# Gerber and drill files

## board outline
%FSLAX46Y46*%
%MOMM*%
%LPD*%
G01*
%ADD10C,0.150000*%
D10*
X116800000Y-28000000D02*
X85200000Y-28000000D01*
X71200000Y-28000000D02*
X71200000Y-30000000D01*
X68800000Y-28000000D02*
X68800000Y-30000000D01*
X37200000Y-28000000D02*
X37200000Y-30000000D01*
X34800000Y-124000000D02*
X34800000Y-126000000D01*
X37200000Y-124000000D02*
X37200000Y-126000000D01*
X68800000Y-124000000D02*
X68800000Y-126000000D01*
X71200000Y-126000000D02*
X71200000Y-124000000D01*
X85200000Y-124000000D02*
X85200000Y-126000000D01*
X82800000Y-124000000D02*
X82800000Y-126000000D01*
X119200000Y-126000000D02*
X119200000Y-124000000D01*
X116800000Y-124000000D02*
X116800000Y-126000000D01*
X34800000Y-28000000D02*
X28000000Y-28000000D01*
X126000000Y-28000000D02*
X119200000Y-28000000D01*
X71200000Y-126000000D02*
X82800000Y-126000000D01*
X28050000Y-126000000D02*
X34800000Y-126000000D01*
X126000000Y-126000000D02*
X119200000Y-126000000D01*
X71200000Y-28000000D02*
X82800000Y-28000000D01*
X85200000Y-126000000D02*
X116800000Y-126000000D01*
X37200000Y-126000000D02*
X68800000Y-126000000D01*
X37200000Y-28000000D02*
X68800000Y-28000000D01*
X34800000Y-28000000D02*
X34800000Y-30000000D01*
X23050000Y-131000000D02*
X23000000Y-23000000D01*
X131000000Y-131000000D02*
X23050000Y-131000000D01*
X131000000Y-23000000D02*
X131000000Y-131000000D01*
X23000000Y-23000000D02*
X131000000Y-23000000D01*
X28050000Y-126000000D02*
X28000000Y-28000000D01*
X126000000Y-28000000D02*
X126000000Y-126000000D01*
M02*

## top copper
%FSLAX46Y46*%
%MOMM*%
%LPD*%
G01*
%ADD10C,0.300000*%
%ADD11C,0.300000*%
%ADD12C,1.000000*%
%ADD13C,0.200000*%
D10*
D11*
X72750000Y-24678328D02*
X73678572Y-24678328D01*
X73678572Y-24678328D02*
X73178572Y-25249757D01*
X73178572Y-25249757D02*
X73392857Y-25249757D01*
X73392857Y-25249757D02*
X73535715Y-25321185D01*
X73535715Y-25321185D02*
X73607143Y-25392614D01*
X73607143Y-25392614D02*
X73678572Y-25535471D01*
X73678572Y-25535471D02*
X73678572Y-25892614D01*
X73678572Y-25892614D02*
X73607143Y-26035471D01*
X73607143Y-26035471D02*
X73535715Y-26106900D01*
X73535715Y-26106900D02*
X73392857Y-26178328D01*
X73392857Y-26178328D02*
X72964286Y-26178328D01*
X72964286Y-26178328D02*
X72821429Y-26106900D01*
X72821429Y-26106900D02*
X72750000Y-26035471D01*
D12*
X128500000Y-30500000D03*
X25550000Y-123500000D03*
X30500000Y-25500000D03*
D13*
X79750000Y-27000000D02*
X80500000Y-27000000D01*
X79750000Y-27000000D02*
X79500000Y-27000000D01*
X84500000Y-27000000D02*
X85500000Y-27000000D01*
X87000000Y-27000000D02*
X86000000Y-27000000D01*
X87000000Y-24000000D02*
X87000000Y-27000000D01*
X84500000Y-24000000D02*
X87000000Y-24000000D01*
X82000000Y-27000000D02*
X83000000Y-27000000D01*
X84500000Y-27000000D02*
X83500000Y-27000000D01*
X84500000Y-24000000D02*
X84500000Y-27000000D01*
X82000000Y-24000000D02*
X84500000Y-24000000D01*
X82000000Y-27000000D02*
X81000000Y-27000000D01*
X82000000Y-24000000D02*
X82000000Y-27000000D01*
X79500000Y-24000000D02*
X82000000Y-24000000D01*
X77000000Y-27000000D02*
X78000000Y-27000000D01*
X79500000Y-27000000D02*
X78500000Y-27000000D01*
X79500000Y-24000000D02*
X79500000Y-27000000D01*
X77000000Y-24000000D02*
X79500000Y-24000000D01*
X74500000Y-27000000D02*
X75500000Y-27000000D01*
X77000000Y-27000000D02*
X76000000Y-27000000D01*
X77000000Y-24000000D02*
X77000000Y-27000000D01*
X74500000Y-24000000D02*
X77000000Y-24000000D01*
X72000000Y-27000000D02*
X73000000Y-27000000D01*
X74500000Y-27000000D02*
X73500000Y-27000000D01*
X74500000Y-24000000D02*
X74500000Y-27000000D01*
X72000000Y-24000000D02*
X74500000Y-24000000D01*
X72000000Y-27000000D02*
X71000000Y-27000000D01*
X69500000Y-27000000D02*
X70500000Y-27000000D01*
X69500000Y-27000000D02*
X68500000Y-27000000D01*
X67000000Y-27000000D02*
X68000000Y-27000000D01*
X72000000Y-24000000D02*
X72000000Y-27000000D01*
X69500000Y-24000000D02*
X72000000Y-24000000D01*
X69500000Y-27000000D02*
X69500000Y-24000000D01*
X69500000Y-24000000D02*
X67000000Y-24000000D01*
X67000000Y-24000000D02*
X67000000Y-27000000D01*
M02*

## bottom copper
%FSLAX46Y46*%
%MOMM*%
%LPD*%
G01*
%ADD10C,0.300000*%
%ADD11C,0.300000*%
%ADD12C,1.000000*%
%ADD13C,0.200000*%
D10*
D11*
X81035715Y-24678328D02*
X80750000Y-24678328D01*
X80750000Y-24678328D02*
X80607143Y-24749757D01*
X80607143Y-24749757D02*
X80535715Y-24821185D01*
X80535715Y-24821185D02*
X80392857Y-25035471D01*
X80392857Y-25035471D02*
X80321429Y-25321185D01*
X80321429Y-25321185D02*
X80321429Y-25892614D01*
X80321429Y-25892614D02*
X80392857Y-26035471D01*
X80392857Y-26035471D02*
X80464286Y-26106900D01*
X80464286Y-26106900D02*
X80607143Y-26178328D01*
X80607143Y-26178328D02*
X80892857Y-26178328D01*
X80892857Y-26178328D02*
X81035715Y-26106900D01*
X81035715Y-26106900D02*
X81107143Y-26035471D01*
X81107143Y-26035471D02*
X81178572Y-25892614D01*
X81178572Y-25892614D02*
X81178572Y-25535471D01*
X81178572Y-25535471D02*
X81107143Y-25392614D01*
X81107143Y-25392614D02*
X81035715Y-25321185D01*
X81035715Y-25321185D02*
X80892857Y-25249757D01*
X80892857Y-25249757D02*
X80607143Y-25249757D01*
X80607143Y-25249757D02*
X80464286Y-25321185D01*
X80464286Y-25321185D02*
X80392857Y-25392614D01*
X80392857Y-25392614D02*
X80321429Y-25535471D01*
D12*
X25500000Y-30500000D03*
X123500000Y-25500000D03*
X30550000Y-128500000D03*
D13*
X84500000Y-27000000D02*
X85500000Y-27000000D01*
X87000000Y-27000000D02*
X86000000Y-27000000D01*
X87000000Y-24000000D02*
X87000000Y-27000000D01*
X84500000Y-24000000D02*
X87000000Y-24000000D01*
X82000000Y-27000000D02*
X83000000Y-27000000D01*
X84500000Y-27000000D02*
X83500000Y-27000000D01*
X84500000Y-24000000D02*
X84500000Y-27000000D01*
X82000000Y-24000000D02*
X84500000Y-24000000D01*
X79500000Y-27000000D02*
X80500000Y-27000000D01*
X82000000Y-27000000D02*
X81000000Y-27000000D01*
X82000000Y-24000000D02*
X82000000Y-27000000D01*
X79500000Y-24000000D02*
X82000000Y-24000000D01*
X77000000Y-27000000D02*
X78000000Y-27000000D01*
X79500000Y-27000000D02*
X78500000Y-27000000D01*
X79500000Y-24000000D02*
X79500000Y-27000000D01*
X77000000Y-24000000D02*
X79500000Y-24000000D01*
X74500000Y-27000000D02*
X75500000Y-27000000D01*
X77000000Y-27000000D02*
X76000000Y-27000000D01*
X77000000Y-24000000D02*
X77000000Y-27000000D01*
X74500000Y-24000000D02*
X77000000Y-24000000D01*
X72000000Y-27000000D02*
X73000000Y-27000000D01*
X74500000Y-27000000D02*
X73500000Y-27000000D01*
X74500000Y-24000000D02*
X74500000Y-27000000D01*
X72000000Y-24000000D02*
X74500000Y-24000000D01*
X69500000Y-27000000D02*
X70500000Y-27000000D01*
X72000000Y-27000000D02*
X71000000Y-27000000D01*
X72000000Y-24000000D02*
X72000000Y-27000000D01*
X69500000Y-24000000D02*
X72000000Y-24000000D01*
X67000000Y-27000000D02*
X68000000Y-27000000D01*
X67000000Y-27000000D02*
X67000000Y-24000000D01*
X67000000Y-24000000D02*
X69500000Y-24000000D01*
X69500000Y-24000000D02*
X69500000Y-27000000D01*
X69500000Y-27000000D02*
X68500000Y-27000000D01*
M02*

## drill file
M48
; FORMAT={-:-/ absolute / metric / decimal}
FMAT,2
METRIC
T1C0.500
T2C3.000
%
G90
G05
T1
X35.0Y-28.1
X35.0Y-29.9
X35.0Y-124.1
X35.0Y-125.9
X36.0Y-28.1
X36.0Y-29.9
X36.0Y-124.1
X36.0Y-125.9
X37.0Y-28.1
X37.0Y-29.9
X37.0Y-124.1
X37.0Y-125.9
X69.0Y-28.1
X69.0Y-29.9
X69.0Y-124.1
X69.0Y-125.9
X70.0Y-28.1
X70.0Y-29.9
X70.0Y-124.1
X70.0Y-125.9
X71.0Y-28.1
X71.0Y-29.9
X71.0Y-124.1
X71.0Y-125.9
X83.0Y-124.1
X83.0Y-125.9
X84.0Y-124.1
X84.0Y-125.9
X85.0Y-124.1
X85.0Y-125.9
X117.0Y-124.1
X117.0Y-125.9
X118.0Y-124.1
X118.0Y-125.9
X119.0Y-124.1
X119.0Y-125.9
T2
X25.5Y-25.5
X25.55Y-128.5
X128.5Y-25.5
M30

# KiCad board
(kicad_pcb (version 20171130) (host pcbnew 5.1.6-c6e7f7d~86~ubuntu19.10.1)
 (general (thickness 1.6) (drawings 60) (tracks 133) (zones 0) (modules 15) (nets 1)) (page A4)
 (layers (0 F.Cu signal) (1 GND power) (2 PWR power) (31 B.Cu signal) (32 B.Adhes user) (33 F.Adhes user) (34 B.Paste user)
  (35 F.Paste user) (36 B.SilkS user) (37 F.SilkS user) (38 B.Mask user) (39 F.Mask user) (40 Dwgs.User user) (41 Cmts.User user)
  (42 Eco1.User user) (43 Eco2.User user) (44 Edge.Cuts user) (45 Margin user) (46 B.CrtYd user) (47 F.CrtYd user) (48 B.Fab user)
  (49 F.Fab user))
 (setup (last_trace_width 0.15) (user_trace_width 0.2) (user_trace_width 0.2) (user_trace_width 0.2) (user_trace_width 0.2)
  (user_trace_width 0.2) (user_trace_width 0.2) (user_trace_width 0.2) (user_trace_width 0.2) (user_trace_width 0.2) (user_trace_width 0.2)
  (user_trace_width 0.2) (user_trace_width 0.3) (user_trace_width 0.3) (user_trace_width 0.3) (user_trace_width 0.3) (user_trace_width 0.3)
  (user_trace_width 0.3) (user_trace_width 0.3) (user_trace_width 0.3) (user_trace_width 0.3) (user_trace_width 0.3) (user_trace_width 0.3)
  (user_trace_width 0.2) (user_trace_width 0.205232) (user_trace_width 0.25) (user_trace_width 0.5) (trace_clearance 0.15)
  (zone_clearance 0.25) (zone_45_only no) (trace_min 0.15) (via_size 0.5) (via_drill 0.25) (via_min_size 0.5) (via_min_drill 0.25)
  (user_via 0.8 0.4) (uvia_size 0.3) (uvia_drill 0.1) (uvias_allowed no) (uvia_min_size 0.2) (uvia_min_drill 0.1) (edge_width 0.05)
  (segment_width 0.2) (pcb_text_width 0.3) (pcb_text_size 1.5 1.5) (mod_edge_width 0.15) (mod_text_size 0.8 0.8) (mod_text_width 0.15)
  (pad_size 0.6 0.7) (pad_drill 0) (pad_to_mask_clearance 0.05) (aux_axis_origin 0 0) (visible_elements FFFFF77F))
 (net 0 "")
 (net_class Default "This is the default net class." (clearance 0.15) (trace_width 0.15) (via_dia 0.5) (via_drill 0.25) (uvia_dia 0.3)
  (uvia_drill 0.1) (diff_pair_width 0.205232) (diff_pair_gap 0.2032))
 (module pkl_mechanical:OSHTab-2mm (layer F.Cu) (at 36 125)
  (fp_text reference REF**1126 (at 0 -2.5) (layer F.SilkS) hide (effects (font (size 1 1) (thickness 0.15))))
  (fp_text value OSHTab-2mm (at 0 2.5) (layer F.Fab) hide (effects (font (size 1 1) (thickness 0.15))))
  (pad "" np_thru_hole circle (at 1 0.9) (size 0.5 0.5) (drill 0.5) (layers *.Cu))
  (pad "" np_thru_hole circle (at 0 0.9) (size 0.5 0.5) (drill 0.5) (layers *.Cu))
  (pad "" np_thru_hole circle (at -1 0.9) (size 0.5 0.5) (drill 0.5) (layers *.Cu))
  (pad "" np_thru_hole circle (at 1 -0.9) (size 0.5 0.5) (drill 0.5) (layers *.Cu))
  (pad "" np_thru_hole circle (at -1 -0.9) (size 0.5 0.5) (drill 0.5) (layers *.Cu))
  (pad "" np_thru_hole circle (at 0 -0.9) (size 0.5 0.5) (drill 0.5) (layers *.Cu)))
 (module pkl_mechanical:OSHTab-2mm (layer F.Cu) (at 70 125)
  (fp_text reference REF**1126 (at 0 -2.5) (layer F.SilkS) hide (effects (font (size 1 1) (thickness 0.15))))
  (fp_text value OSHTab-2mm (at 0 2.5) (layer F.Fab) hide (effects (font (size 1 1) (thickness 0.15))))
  (pad "" np_thru_hole circle (at 1 0.9) (size 0.5 0.5) (drill 0.5) (layers *.Cu))
  (pad "" np_thru_hole circle (at 0 0.9) (size 0.5 0.5) (drill 0.5) (layers *.Cu))
  (pad "" np_thru_hole circle (at -1 0.9) (size 0.5 0.5) (drill 0.5) (layers *.Cu))
  (pad "" np_thru_hole circle (at 1 -0.9) (size 0.5 0.5) (drill 0.5) (layers *.Cu))
  (pad "" np_thru_hole circle (at -1 -0.9) (size 0.5 0.5) (drill 0.5) (layers *.Cu))
  (pad "" np_thru_hole circle (at 0 -0.9) (size 0.5 0.5) (drill 0.5) (layers *.Cu)))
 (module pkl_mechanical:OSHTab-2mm (layer F.Cu) (at 84 125)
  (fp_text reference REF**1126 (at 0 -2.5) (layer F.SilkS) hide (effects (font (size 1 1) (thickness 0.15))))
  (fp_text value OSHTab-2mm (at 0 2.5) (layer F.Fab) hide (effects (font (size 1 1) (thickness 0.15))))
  (pad "" np_thru_hole circle (at 1 0.9) (size 0.5 0.5) (drill 0.5) (layers *.Cu))
  (pad "" np_thru_hole circle (at 0 0.9) (size 0.5 0.5) (drill 0.5) (layers *.Cu))
  (pad "" np_thru_hole circle (at -1 0.9) (size 0.5 0.5) (drill 0.5) (layers *.Cu))
  (pad "" np_thru_hole circle (at 1 -0.9) (size 0.5 0.5) (drill 0.5) (layers *.Cu))
  (pad "" np_thru_hole circle (at -1 -0.9) (size 0.5 0.5) (drill 0.5) (layers *.Cu))
  (pad "" np_thru_hole circle (at 0 -0.9) (size 0.5 0.5) (drill 0.5) (layers *.Cu)))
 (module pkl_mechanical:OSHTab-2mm (layer F.Cu) (at 118 125)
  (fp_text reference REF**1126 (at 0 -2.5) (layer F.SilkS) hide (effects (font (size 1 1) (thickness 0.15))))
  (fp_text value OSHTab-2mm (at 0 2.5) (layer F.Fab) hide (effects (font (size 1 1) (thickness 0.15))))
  (pad "" np_thru_hole circle (at 1 0.9) (size 0.5 0.5) (drill 0.5) (layers *.Cu))
  (pad "" np_thru_hole circle (at 0 0.9) (size 0.5 0.5) (drill 0.5) (layers *.Cu))
  (pad "" np_thru_hole circle (at -1 0.9) (size 0.5 0.5) (drill 0.5) (layers *.Cu))
  (pad "" np_thru_hole circle (at 1 -0.9) (size 0.5 0.5) (drill 0.5) (layers *.Cu))
  (pad "" np_thru_hole circle (at -1 -0.9) (size 0.5 0.5) (drill 0.5) (layers *.Cu))
  (pad "" np_thru_hole circle (at 0 -0.9) (size 0.5 0.5) (drill 0.5) (layers *.Cu)))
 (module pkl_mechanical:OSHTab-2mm (layer F.Cu) (at 70 29)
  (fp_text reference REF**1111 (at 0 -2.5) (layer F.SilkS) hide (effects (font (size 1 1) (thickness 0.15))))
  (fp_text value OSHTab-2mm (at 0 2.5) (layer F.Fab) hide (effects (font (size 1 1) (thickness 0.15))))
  (pad "" np_thru_hole circle (at 1 0.9) (size 0.5 0.5) (drill 0.5) (layers *.Cu))
  (pad "" np_thru_hole circle (at 0 0.9) (size 0.5 0.5) (drill 0.5) (layers *.Cu))
  (pad "" np_thru_hole circle (at -1 0.9) (size 0.5 0.5) (drill 0.5) (layers *.Cu))
  (pad "" np_thru_hole circle (at 1 -0.9) (size 0.5 0.5) (drill 0.5) (layers *.Cu))
  (pad "" np_thru_hole circle (at -1 -0.9) (size 0.5 0.5) (drill 0.5) (layers *.Cu))
  (pad "" np_thru_hole circle (at 0 -0.9) (size 0.5 0.5) (drill 0.5) (layers *.Cu)))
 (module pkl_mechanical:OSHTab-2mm (layer F.Cu) (at 36 29)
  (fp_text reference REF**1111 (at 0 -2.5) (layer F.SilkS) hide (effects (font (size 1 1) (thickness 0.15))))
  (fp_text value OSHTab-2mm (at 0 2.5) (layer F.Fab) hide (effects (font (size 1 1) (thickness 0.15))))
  (pad "" np_thru_hole circle (at 1 0.9) (size 0.5 0.5) (drill 0.5) (layers *.Cu))
  (pad "" np_thru_hole circle (at 0 0.9) (size 0.5 0.5) (drill 0.5) (layers *.Cu))
  (pad "" np_thru_hole circle (at -1 0.9) (size 0.5 0.5) (drill 0.5) (layers *.Cu))
  (pad "" np_thru_hole circle (at 1 -0.9) (size 0.5 0.5) (drill 0.5) (layers *.Cu))
  (pad "" np_thru_hole circle (at -1 -0.9) (size 0.5 0.5) (drill 0.5) (layers *.Cu))
  (pad "" np_thru_hole circle (at 0 -0.9) (size 0.5 0.5) (drill 0.5) (layers *.Cu)))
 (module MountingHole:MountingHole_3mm (layer F.Cu) (at 25.5 25.5)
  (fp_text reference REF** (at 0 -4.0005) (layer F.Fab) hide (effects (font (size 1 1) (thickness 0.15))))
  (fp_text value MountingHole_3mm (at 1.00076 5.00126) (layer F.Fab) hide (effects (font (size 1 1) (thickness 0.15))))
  (pad 1 np_thru_hole circle (at 0 0) (size 3 3) (drill 3) (layers *.Cu *.Mask)))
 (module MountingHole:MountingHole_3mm (layer F.Cu) (at 25.55 128.5)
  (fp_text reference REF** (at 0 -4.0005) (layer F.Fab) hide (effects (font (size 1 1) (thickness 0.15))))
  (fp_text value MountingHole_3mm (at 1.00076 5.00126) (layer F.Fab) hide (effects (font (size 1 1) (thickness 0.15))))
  (pad 1 np_thru_hole circle (at 0 0) (size 3 3) (drill 3) (layers *.Cu *.Mask)))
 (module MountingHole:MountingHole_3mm (layer F.Cu) (at 128.5 25.5)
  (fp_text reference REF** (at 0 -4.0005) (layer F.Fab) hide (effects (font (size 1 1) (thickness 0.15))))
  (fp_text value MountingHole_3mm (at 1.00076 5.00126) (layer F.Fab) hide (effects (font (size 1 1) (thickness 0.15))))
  (pad 1 np_thru_hole circle (at 0 0) (size 3 3) (drill 3) (layers *.Cu *.Mask)))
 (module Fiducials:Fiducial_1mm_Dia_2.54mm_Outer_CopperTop (layer B.Cu) (at 25.5 30.5)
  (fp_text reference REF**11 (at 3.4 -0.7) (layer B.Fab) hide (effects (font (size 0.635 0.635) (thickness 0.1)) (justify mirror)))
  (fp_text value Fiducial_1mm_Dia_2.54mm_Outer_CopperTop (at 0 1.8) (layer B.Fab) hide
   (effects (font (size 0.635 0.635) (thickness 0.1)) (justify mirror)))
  (pad ~ smd circle (at 0 0) (size 1 1) (layers B.Cu B.Mask) (solder_mask_margin 0.77) (clearance 0.77)))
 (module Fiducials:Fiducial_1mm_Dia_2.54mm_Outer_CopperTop (layer B.Cu) (at 123.5 25.5)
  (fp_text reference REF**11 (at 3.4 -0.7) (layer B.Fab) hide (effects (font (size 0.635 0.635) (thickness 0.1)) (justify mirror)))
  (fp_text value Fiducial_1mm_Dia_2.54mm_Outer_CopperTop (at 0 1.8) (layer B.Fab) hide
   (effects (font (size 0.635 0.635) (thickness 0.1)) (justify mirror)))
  (pad ~ smd circle (at 0 0) (size 1 1) (layers B.Cu B.Mask) (solder_mask_margin 0.77) (clearance 0.77)))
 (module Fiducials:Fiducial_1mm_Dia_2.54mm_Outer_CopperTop (layer B.Cu) (at 30.55 128.5)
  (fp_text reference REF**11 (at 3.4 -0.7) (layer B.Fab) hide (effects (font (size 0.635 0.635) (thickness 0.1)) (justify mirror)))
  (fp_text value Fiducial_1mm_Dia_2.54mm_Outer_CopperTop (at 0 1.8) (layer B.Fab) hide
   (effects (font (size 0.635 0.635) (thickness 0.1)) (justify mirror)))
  (pad ~ smd circle (at 0 0) (size 1 1) (layers B.Cu B.Mask) (solder_mask_margin 0.77) (clearance 0.77)))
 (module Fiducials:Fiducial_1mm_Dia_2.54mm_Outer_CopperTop (layer F.Cu) (at 128.5 30.5)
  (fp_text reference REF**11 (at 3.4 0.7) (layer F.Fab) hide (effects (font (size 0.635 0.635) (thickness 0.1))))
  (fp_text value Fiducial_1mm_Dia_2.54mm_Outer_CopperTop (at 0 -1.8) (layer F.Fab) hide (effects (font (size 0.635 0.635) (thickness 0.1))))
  (pad ~ smd circle (at 0 0) (size 1 1) (layers F.Cu F.Mask) (solder_mask_margin 0.77) (clearance 0.77)))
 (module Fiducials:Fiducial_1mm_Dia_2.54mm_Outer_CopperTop (layer F.Cu) (at 25.55 123.5)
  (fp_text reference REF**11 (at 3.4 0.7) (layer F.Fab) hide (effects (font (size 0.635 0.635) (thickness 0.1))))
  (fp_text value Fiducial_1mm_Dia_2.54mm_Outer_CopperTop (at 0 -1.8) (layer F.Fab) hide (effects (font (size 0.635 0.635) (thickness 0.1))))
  (pad ~ smd circle (at 0 0) (size 1 1) (layers F.Cu F.Mask) (solder_mask_margin 0.77) (clearance 0.77)))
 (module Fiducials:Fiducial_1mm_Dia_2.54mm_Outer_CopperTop (layer F.Cu) (at 30.5 25.5)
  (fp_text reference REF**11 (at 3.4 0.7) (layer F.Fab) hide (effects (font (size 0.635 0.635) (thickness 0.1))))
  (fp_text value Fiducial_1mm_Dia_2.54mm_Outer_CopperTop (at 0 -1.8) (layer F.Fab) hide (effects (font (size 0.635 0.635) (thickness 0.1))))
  (pad ~ smd circle (at 0 0) (size 1 1) (layers F.Cu F.Mask) (solder_mask_margin 0.77) (clearance 0.77)))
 (gr_line (start 116.8 28) (end 85.2 28) (layer Edge.Cuts) (width 0.15))
 (gr_line (start 71.2 28) (end 71.2 30) (layer Edge.Cuts) (width 0.15))
 (gr_line (start 68.8 28) (end 68.8 30) (layer Edge.Cuts) (width 0.15))
 (gr_line (start 37.2 28) (end 37.2 30) (layer Edge.Cuts) (width 0.15))
 (gr_line (start 34.8 124) (end 34.8 126) (layer Edge.Cuts) (width 0.15))
 (gr_line (start 37.2 124) (end 37.2 126) (layer Edge.Cuts) (width 0.15))
 (gr_line (start 68.8 124) (end 68.8 126) (layer Edge.Cuts) (width 0.15))
 (gr_line (start 71.2 126) (end 71.2 124) (layer Edge.Cuts) (width 0.15))
 (gr_line (start 85.2 124) (end 85.2 126) (layer Edge.Cuts) (width 0.15))
 (gr_line (start 82.8 124) (end 82.8 126) (layer Edge.Cuts) (width 0.15))
 (gr_line (start 119.2 126) (end 119.2 124) (layer Edge.Cuts) (width 0.15))
 (gr_line (start 116.8 124) (end 116.8 126) (layer Edge.Cuts) (width 0.15))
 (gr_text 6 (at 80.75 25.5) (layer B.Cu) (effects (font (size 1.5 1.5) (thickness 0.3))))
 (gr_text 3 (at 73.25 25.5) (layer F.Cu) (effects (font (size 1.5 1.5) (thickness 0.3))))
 (gr_line (start 34.8 28) (end 28 28) (layer Edge.Cuts) (width 0.15))
 (gr_line (start 126 28) (end 119.2 28) (layer Edge.Cuts) (width 0.15))
 (gr_line (start 71.2 126) (end 82.8 126) (layer Edge.Cuts) (width 0.15))
 (gr_line (start 28.05 126) (end 34.8 126) (layer Edge.Cuts) (width 0.15))
 (gr_line (start 126 126) (end 119.2 126) (layer Edge.Cuts) (width 0.15))
 (gr_line (start 71.2 28) (end 82.8 28) (layer Edge.Cuts) (width 0.15))
 (gr_line (start 85.2 126) (end 116.8 126) (layer Edge.Cuts) (width 0.15))
 (gr_line (start 37.2 126) (end 68.8 126) (layer Edge.Cuts) (width 0.15))
 (gr_line (start 37.2 28) (end 68.8 28) (layer Edge.Cuts) (width 0.15))
 (gr_line (start 34.8 28) (end 34.8 30) (layer Edge.Cuts) (width 0.15))
 (gr_line (start 23.05 131) (end 23 23) (layer Edge.Cuts) (width 0.15))
 (gr_line (start 131 131) (end 23.05 131) (layer Edge.Cuts) (width 0.15))
 (gr_line (start 131 23) (end 131 131) (layer Edge.Cuts) (width 0.15))
 (gr_line (start 23 23) (end 131 23) (layer Edge.Cuts) (width 0.15))
 (gr_line (start 28.05 126) (end 28 28) (layer Edge.Cuts) (width 0.15))
 (gr_line (start 126 28) (end 126 126) (layer Edge.Cuts) (width 0.15))
 (segment (start 84.5 27) (end 85.5 27) (width 0.2) (layer B.Cu) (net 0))
 (segment (start 87 27) (end 86 27) (width 0.2) (layer B.Cu) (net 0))
 (segment (start 87 24) (end 87 27) (width 0.2) (layer B.Cu) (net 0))
 (segment (start 84.5 24) (end 87 24) (width 0.2) (layer B.Cu) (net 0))
 (segment (start 82 27) (end 83 27) (width 0.2) (layer B.Cu) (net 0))
 (segment (start 84.5 27) (end 83.5 27) (width 0.2) (layer B.Cu) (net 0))
 (segment (start 84.5 24) (end 84.5 27) (width 0.2) (layer B.Cu) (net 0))
 (segment (start 82 24) (end 84.5 24) (width 0.2) (layer B.Cu) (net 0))
 (segment (start 79.5 27) (end 80.5 27) (width 0.2) (layer B.Cu) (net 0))
 (segment (start 82 27) (end 81 27) (width 0.2) (layer B.Cu) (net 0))
 (segment (start 82 24) (end 82 27) (width 0.2) (layer B.Cu) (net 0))
 (segment (start 79.5 24) (end 82 24) (width 0.2) (layer B.Cu) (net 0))
 (segment (start 77 27) (end 78 27) (width 0.2) (layer B.Cu) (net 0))
 (segment (start 79.5 27) (end 78.5 27) (width 0.2) (layer B.Cu) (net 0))
 (segment (start 79.5 24) (end 79.5 27) (width 0.2) (layer B.Cu) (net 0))
 (segment (start 77 24) (end 79.5 24) (width 0.2) (layer B.Cu) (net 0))
 (segment (start 74.5 27) (end 75.5 27) (width 0.2) (layer B.Cu) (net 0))
 (segment (start 77 27) (end 76 27) (width 0.2) (layer B.Cu) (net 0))
 (segment (start 77 24) (end 77 27) (width 0.2) (layer B.Cu) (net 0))
 (segment (start 74.5 24) (end 77 24) (width 0.2) (layer B.Cu) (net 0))
 (segment (start 72 27) (end 73 27) (width 0.2) (layer B.Cu) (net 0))
 (segment (start 74.5 27) (end 73.5 27) (width 0.2) (layer B.Cu) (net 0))
 (segment (start 74.5 24) (end 74.5 27) (width 0.2) (layer B.Cu) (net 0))
 (segment (start 72 24) (end 74.5 24) (width 0.2) (layer B.Cu) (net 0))
 (segment (start 69.5 27) (end 70.5 27) (width 0.2) (layer B.Cu) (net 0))
 (segment (start 72 27) (end 71 27) (width 0.2) (layer B.Cu) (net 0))
 (segment (start 72 24) (end 72 27) (width 0.2) (layer B.Cu) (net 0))
 (segment (start 69.5 24) (end 72 24) (width 0.2) (layer B.Cu) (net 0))
 (segment (start 67 27) (end 68 27) (width 0.2) (layer B.Cu) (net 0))
 (segment (start 67 27) (end 67 24) (width 0.2) (layer B.Cu) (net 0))
 (segment (start 67 24) (end 69.5 24) (width 0.2) (layer B.Cu) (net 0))
 (segment (start 69.5 24) (end 69.5 27) (width 0.2) (layer B.Cu) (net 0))
 (segment (start 69.5 27) (end 68.5 27) (width 0.2) (layer B.Cu) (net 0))
 (segment (start 84.5 27) (end 85.5 27) (width 0.2) (layer PWR) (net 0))
 (segment (start 87 27) (end 86 27) (width 0.2) (layer PWR) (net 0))
 (segment (start 87 24) (end 87 27) (width 0.2) (layer PWR) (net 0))
 (segment (start 84.5 24) (end 87 24) (width 0.2) (layer PWR) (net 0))
 (segment (start 82 27) (end 83 27) (width 0.2) (layer PWR) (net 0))
 (segment (start 84.5 27) (end 83.5 27) (width 0.2) (layer PWR) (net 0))
 (segment (start 84.5 24) (end 84.5 27) (width 0.2) (layer PWR) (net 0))
 (segment (start 82 24) (end 84.5 24) (width 0.2) (layer PWR) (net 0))
 (segment (start 79.5 27) (end 80.5 27) (width 0.2) (layer PWR) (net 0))
 (segment (start 79.75 27) (end 80.5 27) (width 0.2) (layer F.Cu) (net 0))
 (segment (start 79.75 27) (end 79.5 27) (width 0.2) (layer F.Cu) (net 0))
 (segment (start 82 27) (end 81 27) (width 0.2) (layer PWR) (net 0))
 (segment (start 82 24) (end 82 27) (width 0.2) (layer PWR) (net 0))
 (segment (start 79.5 24) (end 82 24) (width 0.2) (layer PWR) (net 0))
 (segment (start 77 27) (end 78 27) (width 0.2) (layer PWR) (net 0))
 (segment (start 79.5 27) (end 78.5 27) (width 0.2) (layer PWR) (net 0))
 (segment (start 79.5 24) (end 79.5 27) (width 0.2) (layer PWR) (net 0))
 (segment (start 77 24) (end 79.5 24) (width 0.2) (layer PWR) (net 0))
 (segment (start 74.5 27) (end 75.5 27) (width 0.2) (layer PWR) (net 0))
 (segment (start 77 27) (end 76 27) (width 0.2) (layer PWR) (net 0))
 (segment (start 77 24) (end 77 27) (width 0.2) (layer PWR) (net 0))
 (segment (start 74.5 24) (end 77 24) (width 0.2) (layer PWR) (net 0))
 (segment (start 72 27) (end 73 27) (width 0.2) (layer PWR) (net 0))
 (segment (start 74.5 27) (end 73.5 27) (width 0.2) (layer PWR) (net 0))
 (segment (start 74.5 24) (end 74.5 27) (width 0.2) (layer PWR) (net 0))
 (segment (start 72 24) (end 74.5 24) (width 0.2) (layer PWR) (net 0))
 (segment (start 69.5 27) (end 70.5 27) (width 0.2) (layer PWR) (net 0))
 (segment (start 72 27) (end 71 27) (width 0.2) (layer PWR) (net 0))
 (segment (start 72 24) (end 72 27) (width 0.2) (layer PWR) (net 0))
 (segment (start 69.5 24) (end 72 24) (width 0.2) (layer PWR) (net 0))
 (segment (start 67 27) (end 68 27) (width 0.2) (layer PWR) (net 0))
 (segment (start 67 27) (end 67 24) (width 0.2) (layer PWR) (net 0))
 (segment (start 67 24) (end 69.5 24) (width 0.2) (layer PWR) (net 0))
 (segment (start 69.5 24) (end 69.5 27) (width 0.2) (layer PWR) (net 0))
 (segment (start 69.5 27) (end 68.5 27) (width 0.2) (layer PWR) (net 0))
 (segment (start 84.5 27) (end 85.5 27) (width 0.2) (layer GND) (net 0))
 (segment (start 87 27) (end 86 27) (width 0.2) (layer GND) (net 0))
 (segment (start 87 24) (end 87 27) (width 0.2) (layer GND) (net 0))
 (segment (start 84.5 24) (end 87 24) (width 0.2) (layer GND) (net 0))
 (segment (start 82 27) (end 83 27) (width 0.2) (layer GND) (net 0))
 (segment (start 84.5 27) (end 83.5 27) (width 0.2) (layer GND) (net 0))
 (segment (start 84.5 24) (end 84.5 27) (width 0.2) (layer GND) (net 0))
 (segment (start 82 24) (end 84.5 24) (width 0.2) (layer GND) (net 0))
 (segment (start 79.5 27) (end 80.5 27) (width 0.2) (layer GND) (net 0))
 (segment (start 82 27) (end 81 27) (width 0.2) (layer GND) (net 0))
 (segment (start 82 24) (end 82 27) (width 0.2) (layer GND) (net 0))
 (segment (start 79.5 24) (end 82 24) (width 0.2) (layer GND) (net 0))
 (segment (start 77 27) (end 78 27) (width 0.2) (layer GND) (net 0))
 (segment (start 79.5 27) (end 78.5 27) (width 0.2) (layer GND) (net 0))
 (segment (start 79.5 24) (end 79.5 27) (width 0.2) (layer GND) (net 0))
 (segment (start 77 24) (end 79.5 24) (width 0.2) (layer GND) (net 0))
 (segment (start 74.5 27) (end 75.5 27) (width 0.2) (layer GND) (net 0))
 (segment (start 77 27) (end 76 27) (width 0.2) (layer GND) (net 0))
 (segment (start 77 24) (end 77 27) (width 0.2) (layer GND) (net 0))
 (segment (start 74.5 24) (end 77 24) (width 0.2) (layer GND) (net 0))
 (segment (start 72 27) (end 73 27) (width 0.2) (layer GND) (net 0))
 (segment (start 74.5 27) (end 73.5 27) (width 0.2) (layer GND) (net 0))
 (segment (start 74.5 24) (end 74.5 27) (width 0.2) (layer GND) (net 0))
 (segment (start 72 24) (end 74.5 24) (width 0.2) (layer GND) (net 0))
 (segment (start 69.5 27) (end 70.5 27) (width 0.2) (layer GND) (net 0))
 (segment (start 72 27) (end 71 27) (width 0.2) (layer GND) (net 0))
 (segment (start 72 24) (end 72 27) (width 0.2) (layer GND) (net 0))
 (segment (start 69.5 24) (end 72 24) (width 0.2) (layer GND) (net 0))
 (segment (start 67 27) (end 68 27) (width 0.2) (layer GND) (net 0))
 (segment (start 67 24) (end 67 27) (width 0.2) (layer GND) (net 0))
 (segment (start 67 24) (end 69.5 24) (width 0.2) (layer GND) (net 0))
 (segment (start 69.5 24) (end 69.5 27) (width 0.2) (layer GND) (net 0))
 (segment (start 69.5 27) (end 68.5 27) (width 0.2) (layer GND) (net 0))
 (segment (start 84.5 27) (end 85.5 27) (width 0.2) (layer F.Cu) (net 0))
 (segment (start 87 27) (end 86 27) (width 0.2) (layer F.Cu) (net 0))
 (segment (start 87 24) (end 87 27) (width 0.2) (layer F.Cu) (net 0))
 (segment (start 84.5 24) (end 87 24) (width 0.2) (layer F.Cu) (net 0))
 (segment (start 82 27) (end 83 27) (width 0.2) (layer F.Cu) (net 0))
 (segment (start 84.5 27) (end 83.5 27) (width 0.2) (layer F.Cu) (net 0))
 (segment (start 84.5 24) (end 84.5 27) (width 0.2) (layer F.Cu) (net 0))
 (segment (start 82 24) (end 84.5 24) (width 0.2) (layer F.Cu) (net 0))
 (segment (start 82 27) (end 81 27) (width 0.2) (layer F.Cu) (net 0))
 (segment (start 82 24) (end 82 27) (width 0.2) (layer F.Cu) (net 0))
 (segment (start 79.5 24) (end 82 24) (width 0.2) (layer F.Cu) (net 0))
 (segment (start 77 27) (end 78 27) (width 0.2) (layer F.Cu) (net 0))
 (segment (start 79.5 27) (end 78.5 27) (width 0.2) (layer F.Cu) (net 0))
 (segment (start 79.5 24) (end 79.5 27) (width 0.2) (layer F.Cu) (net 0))
 (segment (start 77 24) (end 79.5 24) (width 0.2) (layer F.Cu) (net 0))
 (segment (start 74.5 27) (end 75.5 27) (width 0.2) (layer F.Cu) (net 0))
 (segment (start 77 27) (end 76 27) (width 0.2) (layer F.Cu) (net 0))
 (segment (start 77 24) (end 77 27) (width 0.2) (layer F.Cu) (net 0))
 (segment (start 74.5 24) (end 77 24) (width 0.2) (layer F.Cu) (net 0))
 (segment (start 72 27) (end 73 27) (width 0.2) (layer F.Cu) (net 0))
 (segment (start 74.5 27) (end 73.5 27) (width 0.2) (layer F.Cu) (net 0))
 (segment (start 74.5 24) (end 74.5 27) (width 0.2) (layer F.Cu) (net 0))
 (segment (start 72 24) (end 74.5 24) (width 0.2) (layer F.Cu) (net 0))
 (segment (start 72 27) (end 71 27) (width 0.2) (layer F.Cu) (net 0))
 (segment (start 69.5 27) (end 70.5 27) (width 0.2) (layer F.Cu) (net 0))
 (segment (start 69.5 27) (end 68.5 27) (width 0.2) (layer F.Cu) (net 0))
 (segment (start 67 27) (end 68 27) (width 0.2) (layer F.Cu) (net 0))
 (segment (start 72 24) (end 72 27) (width 0.2) (layer F.Cu) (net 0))
 (segment (start 69.5 24) (end 72 24) (width 0.2) (layer F.Cu) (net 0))
 (segment (start 69.5 27) (end 69.5 24) (width 0.2) (layer F.Cu) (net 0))
 (segment (start 69.5 24) (end 67 24) (width 0.2) (layer F.Cu) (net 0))
 (segment (start 67 24) (end 67 27) (width 0.2) (layer F.Cu) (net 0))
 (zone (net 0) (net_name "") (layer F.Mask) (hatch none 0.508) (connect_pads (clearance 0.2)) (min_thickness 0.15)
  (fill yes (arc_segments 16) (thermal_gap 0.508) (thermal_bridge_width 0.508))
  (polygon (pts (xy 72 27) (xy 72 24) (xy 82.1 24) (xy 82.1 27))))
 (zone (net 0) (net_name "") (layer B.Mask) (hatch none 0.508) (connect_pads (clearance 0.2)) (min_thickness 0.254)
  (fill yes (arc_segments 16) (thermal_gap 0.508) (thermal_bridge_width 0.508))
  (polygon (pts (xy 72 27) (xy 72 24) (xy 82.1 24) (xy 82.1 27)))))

